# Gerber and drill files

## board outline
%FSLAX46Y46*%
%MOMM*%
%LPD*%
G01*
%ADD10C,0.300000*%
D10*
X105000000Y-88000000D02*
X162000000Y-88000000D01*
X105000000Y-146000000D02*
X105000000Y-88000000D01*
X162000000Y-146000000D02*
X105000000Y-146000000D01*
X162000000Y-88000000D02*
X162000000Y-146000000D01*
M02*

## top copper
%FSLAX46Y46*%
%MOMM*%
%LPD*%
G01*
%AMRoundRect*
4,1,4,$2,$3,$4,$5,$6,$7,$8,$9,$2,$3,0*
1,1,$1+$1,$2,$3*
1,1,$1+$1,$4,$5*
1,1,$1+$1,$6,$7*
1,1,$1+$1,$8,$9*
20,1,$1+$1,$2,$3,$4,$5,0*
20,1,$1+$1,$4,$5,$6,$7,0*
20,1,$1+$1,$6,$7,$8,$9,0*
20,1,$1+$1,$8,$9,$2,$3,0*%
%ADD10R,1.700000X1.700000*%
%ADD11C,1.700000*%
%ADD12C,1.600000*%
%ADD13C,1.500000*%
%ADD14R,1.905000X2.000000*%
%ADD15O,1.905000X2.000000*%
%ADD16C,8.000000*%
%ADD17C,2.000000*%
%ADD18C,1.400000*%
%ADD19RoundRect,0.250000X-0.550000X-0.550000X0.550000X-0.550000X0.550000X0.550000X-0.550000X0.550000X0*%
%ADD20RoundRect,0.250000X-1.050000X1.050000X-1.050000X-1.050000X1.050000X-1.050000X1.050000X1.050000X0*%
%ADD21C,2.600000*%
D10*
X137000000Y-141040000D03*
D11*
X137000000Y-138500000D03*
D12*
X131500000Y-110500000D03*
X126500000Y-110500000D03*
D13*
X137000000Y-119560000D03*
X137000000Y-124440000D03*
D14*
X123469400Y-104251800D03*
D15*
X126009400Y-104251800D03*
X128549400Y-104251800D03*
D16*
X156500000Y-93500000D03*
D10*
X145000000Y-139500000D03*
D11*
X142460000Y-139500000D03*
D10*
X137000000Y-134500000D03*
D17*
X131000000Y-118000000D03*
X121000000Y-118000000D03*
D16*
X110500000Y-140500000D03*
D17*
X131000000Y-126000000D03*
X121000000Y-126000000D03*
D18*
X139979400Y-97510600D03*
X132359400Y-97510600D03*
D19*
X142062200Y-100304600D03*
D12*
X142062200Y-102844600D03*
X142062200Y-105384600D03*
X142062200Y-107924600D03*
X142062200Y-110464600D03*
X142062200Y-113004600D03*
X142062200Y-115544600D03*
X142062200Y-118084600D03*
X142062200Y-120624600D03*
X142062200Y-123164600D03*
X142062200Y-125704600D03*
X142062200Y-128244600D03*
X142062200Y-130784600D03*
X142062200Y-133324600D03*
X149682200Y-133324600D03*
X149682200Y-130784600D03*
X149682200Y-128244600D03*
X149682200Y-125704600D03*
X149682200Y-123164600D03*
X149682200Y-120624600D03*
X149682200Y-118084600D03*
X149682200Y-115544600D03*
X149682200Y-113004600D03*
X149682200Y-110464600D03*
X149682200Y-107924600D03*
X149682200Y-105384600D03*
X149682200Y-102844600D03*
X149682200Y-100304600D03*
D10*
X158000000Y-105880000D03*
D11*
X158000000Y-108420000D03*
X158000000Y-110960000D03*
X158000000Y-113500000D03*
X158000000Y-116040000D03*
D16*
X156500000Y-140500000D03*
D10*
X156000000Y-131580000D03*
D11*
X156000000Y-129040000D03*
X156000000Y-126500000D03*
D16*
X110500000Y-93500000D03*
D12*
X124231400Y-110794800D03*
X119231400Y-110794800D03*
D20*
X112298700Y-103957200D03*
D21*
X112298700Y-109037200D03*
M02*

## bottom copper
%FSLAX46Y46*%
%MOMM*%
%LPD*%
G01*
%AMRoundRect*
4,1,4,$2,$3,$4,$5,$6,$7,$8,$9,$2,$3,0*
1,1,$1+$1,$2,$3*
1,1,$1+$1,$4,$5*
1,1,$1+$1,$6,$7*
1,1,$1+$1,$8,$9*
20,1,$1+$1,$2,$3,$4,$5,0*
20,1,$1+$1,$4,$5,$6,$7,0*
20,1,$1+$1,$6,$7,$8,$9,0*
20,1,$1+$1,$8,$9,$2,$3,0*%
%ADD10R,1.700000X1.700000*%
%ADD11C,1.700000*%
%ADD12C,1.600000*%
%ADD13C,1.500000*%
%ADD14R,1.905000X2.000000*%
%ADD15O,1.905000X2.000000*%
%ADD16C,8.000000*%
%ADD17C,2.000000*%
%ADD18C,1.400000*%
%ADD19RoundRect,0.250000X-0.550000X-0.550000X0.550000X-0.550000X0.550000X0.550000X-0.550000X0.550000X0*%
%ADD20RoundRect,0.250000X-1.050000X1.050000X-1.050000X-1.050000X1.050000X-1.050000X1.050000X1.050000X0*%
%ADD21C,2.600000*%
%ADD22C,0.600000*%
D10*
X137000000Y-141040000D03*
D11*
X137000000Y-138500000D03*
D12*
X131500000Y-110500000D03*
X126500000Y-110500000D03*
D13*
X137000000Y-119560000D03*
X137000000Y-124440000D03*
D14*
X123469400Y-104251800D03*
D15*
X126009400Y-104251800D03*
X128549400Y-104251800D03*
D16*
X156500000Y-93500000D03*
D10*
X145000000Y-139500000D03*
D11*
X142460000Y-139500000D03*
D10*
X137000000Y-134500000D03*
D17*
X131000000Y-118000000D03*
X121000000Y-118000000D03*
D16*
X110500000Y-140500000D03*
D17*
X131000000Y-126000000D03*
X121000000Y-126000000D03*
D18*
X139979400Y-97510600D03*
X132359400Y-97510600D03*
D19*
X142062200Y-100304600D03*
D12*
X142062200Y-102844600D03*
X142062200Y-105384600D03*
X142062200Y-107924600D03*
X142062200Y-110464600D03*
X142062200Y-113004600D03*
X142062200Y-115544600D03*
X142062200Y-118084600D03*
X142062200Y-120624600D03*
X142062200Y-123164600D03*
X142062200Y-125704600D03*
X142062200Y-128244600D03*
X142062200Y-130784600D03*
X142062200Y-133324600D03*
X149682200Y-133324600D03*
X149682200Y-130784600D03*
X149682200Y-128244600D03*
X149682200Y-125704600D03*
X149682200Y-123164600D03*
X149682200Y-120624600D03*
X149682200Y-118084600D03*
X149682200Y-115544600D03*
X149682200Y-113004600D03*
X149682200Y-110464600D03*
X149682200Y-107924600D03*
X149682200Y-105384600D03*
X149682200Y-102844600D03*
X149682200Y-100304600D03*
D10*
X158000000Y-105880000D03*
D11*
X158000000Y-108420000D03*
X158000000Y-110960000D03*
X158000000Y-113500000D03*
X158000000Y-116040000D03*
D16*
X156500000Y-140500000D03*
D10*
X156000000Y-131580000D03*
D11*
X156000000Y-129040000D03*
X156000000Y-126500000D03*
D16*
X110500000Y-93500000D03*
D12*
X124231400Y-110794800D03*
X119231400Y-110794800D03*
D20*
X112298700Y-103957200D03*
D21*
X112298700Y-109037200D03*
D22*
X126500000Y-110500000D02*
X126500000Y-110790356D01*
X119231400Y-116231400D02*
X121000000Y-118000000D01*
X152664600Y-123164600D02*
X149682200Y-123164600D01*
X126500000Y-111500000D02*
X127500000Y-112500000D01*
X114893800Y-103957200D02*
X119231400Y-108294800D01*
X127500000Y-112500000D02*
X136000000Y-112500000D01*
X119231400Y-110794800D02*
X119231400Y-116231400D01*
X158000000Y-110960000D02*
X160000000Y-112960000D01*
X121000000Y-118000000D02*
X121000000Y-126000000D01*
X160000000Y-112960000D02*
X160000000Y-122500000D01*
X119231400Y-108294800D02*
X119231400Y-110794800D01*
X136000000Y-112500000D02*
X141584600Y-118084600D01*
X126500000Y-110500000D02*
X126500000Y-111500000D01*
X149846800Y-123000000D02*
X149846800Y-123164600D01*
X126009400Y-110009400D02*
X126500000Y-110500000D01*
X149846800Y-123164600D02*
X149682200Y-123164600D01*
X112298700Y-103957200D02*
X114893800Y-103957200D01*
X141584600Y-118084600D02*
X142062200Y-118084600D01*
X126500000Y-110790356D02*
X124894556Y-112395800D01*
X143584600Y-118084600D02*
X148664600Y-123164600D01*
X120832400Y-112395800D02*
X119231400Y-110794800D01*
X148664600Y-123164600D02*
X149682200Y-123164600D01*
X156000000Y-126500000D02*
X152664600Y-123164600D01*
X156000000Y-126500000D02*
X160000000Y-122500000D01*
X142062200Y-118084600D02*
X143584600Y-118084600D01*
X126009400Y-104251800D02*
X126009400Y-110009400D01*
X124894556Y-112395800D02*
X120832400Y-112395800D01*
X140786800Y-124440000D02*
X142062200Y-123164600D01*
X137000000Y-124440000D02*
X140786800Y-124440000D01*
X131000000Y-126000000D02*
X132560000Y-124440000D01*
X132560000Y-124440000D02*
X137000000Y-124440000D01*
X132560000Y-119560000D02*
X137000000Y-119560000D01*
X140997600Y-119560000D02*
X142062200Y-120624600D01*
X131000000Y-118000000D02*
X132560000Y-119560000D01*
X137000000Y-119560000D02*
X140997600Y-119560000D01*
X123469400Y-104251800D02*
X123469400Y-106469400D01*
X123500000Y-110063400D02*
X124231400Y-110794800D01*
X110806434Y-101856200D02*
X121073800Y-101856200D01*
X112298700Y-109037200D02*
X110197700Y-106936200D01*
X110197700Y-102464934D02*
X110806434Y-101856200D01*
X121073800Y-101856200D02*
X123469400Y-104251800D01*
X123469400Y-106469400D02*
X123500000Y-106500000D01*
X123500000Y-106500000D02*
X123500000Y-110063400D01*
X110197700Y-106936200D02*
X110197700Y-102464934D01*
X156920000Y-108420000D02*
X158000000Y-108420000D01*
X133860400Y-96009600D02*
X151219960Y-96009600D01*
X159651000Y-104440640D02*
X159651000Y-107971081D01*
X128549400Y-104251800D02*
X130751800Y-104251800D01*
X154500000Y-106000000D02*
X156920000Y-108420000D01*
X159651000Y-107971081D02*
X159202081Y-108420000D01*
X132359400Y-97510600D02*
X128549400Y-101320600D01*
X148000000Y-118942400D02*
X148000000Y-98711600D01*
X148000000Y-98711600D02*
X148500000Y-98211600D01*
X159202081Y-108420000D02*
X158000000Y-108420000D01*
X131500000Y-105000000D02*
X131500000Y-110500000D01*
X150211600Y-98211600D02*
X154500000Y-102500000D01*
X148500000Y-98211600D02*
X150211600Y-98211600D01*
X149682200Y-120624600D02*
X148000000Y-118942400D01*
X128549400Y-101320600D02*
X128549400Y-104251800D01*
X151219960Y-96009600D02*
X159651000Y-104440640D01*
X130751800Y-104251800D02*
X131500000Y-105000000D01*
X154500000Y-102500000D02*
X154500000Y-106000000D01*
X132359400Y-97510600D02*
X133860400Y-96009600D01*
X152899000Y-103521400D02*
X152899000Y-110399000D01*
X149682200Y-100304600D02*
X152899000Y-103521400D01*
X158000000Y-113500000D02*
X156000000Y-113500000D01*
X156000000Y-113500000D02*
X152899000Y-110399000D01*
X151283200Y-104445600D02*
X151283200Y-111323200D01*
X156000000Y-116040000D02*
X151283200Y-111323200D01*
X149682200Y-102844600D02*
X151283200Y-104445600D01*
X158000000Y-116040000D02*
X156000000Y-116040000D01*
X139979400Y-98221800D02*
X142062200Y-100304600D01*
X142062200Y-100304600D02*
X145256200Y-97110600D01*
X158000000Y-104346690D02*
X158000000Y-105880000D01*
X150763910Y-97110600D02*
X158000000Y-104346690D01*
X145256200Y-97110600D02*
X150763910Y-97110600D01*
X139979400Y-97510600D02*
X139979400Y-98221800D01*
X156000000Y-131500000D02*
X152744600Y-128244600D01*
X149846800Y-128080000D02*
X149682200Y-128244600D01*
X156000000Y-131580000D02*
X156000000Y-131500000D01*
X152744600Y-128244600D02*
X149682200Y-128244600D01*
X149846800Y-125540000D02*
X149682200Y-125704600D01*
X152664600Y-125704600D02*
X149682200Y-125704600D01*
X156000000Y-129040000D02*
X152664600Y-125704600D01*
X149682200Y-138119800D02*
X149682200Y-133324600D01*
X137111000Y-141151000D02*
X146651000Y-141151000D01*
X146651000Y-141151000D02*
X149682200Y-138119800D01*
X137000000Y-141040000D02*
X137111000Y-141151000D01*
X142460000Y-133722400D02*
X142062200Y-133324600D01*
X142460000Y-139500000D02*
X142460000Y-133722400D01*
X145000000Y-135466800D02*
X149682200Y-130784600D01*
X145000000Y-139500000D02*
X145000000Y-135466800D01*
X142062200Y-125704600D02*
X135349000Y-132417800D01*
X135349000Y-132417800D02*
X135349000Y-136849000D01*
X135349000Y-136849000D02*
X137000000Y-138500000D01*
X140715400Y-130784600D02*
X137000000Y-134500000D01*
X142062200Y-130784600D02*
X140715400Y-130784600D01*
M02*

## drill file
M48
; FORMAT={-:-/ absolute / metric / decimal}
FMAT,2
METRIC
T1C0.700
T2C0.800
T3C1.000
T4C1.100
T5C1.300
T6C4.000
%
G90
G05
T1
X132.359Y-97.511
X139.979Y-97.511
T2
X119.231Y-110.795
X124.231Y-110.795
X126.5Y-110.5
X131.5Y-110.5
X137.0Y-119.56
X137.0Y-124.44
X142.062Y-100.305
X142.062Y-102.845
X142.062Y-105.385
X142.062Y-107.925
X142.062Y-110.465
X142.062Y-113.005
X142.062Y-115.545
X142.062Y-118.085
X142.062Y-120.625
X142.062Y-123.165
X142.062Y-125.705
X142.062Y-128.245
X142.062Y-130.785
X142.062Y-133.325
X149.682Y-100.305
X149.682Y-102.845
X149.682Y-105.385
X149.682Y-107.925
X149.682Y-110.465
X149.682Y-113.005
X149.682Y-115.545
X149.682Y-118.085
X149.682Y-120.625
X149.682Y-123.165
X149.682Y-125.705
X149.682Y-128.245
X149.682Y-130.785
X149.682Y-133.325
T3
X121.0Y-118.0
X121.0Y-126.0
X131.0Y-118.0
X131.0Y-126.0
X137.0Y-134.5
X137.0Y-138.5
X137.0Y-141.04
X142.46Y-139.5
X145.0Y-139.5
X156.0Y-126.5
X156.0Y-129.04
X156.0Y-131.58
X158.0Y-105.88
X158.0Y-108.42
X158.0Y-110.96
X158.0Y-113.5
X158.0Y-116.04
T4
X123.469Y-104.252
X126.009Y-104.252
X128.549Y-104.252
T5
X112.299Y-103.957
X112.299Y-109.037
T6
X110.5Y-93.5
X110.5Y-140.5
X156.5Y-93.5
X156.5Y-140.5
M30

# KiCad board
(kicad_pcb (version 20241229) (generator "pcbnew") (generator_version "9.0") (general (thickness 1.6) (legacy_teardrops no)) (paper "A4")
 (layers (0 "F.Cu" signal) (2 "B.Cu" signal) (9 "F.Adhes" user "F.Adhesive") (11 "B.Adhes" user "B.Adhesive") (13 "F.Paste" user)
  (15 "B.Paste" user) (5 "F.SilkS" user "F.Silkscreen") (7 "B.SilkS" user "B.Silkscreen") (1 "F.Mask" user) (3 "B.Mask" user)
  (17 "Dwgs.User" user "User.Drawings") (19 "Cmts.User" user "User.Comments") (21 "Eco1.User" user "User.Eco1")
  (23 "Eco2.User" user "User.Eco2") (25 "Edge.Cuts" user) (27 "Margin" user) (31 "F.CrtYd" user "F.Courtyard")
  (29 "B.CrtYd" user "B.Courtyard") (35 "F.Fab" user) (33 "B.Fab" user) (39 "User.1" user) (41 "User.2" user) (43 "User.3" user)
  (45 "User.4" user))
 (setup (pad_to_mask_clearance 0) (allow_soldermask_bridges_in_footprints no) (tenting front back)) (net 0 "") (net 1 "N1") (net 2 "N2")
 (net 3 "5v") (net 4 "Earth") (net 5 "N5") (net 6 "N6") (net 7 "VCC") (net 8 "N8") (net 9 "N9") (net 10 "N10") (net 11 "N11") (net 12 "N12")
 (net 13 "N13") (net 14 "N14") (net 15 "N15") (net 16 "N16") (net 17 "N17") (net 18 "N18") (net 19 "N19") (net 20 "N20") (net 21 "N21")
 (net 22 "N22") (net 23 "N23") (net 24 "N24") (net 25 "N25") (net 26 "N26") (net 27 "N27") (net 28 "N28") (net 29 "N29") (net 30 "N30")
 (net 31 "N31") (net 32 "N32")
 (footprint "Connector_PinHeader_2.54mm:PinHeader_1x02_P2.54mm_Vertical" (layer "F.Cu") (at 137 141.04 180)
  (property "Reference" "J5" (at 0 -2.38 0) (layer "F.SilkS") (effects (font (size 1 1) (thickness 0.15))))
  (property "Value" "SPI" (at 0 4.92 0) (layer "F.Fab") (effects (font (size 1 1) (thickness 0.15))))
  (pad "1" thru_hole rect (at 0 0 180) (size 1.7 1.7) (drill 1) (layers "*.Cu" "*.Mask") (remove_unused_layers no) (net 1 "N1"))
  (pad "2" thru_hole circle (at 0 2.54 180) (size 1.7 1.7) (drill 1) (layers "*.Cu" "*.Mask") (remove_unused_layers no) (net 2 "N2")))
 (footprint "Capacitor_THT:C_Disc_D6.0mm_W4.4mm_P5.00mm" (layer "F.Cu") (at 131.5 110.5 180)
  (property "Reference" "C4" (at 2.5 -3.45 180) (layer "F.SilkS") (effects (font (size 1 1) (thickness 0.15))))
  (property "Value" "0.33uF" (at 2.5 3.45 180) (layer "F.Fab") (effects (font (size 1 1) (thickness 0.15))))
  (pad "1" thru_hole circle (at 0 0 180) (size 1.6 1.6) (drill 0.8) (layers "*.Cu" "*.Mask") (remove_unused_layers no) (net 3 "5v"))
  (pad "2" thru_hole circle (at 5 0 180) (size 1.6 1.6) (drill 0.8) (layers "*.Cu" "*.Mask") (remove_unused_layers no) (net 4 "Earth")))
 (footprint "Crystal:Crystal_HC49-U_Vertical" (layer "F.Cu") (at 137 119.56 -90)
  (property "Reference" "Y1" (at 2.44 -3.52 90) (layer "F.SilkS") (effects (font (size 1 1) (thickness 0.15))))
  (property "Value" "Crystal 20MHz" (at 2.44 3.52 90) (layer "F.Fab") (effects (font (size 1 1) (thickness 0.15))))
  (pad "1" thru_hole circle (at 0 0 270) (size 1.5 1.5) (drill 0.8) (layers "*.Cu" "*.Mask") (remove_unused_layers no) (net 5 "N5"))
  (pad "2" thru_hole circle (at 4.88 0 270) (size 1.5 1.5) (drill 0.8) (layers "*.Cu" "*.Mask") (remove_unused_layers no) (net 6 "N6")))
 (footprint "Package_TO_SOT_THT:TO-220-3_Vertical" (layer "F.Cu") (at 123.4694 104.2518)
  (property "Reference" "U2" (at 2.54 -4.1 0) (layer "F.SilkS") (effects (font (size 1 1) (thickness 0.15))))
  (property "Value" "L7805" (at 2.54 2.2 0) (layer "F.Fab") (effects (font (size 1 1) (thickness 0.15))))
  (pad "1" thru_hole rect (at 0 0) (size 1.905 2) (drill 1.1) (layers "*.Cu" "*.Mask") (remove_unused_layers no) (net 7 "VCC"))
  (pad "2" thru_hole oval (at 2.54 0) (size 1.905 2) (drill 1.1) (layers "*.Cu" "*.Mask") (remove_unused_layers no) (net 4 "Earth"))
  (pad "3" thru_hole oval (at 5.08 0) (size 1.905 2) (drill 1.1) (layers "*.Cu" "*.Mask") (remove_unused_layers no) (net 3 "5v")))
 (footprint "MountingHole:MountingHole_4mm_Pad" (layer "F.Cu") (at 156.5 93.5)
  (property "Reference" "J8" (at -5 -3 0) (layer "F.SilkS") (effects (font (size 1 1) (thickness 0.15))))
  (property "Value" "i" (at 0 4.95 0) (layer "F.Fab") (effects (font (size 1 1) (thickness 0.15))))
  (pad "1" thru_hole circle (at 0 0) (size 8 8) (drill 4) (layers "*.Cu" "*.Mask") (remove_unused_layers no) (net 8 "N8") (zone_connect 2)))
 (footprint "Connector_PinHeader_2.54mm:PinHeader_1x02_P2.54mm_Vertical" (layer "F.Cu") (at 145 139.5 -90)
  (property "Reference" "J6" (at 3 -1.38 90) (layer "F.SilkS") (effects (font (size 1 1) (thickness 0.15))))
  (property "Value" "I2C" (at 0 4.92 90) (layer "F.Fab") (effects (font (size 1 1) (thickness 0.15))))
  (pad "1" thru_hole rect (at 0 0 270) (size 1.7 1.7) (drill 1) (layers "*.Cu" "*.Mask") (remove_unused_layers no) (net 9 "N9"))
  (pad "2" thru_hole circle (at 0 2.54 270) (size 1.7 1.7) (drill 1) (layers "*.Cu" "*.Mask") (remove_unused_layers no) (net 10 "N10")))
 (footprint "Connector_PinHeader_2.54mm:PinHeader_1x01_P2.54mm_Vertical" (layer "F.Cu") (at 137 134.5)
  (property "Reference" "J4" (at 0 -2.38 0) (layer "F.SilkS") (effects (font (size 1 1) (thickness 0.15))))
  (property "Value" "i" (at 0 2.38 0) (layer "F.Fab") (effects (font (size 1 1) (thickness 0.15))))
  (pad "1" thru_hole rect (at 0 0) (size 1.7 1.7) (drill 1) (layers "*.Cu" "*.Mask") (remove_unused_layers no) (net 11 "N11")))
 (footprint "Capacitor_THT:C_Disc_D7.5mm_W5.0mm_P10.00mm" (layer "F.Cu") (at 131 118 180)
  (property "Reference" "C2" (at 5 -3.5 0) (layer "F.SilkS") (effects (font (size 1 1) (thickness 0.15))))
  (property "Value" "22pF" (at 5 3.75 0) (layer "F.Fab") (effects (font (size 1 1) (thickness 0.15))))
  (pad "1" thru_hole circle (at 0 0 180) (size 2 2) (drill 1) (layers "*.Cu" "*.Mask") (remove_unused_layers no) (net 5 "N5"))
  (pad "2" thru_hole circle (at 10 0 180) (size 2 2) (drill 1) (layers "*.Cu" "*.Mask") (remove_unused_layers no) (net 4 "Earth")))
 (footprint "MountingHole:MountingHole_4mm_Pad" (layer "F.Cu") (at 110.5 140.5)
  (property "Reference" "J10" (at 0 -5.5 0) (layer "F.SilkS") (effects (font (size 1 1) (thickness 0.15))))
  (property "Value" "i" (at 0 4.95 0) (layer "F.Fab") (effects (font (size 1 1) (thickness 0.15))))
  (pad "1" thru_hole circle (at 0 0) (size 8 8) (drill 4) (layers "*.Cu" "*.Mask") (remove_unused_layers no) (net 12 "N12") (zone_connect 2)))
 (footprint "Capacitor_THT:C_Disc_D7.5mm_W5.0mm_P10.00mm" (layer "F.Cu") (at 131 126 180)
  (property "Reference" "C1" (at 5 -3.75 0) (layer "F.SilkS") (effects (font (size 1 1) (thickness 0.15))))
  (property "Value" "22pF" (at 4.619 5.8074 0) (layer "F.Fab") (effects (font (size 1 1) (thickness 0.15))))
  (pad "1" thru_hole circle (at 0 0 180) (size 2 2) (drill 1) (layers "*.Cu" "*.Mask") (remove_unused_layers no) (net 6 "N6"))
  (pad "2" thru_hole circle (at 10 0 180) (size 2 2) (drill 1) (layers "*.Cu" "*.Mask") (remove_unused_layers no) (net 4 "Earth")))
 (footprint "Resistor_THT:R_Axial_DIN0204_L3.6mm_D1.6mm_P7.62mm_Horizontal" (layer "F.Cu") (at 139.9794 97.5106 180)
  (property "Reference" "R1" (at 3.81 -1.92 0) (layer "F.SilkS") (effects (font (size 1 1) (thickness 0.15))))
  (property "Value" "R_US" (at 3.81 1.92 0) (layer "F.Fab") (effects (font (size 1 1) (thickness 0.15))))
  (pad "1" thru_hole circle (at 0 0 180) (size 1.4 1.4) (drill 0.7) (layers "*.Cu" "*.Mask") (remove_unused_layers no) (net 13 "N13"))
  (pad "2" thru_hole circle (at 7.62 0 180) (size 1.4 1.4) (drill 0.7) (layers "*.Cu" "*.Mask") (remove_unused_layers no) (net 3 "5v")))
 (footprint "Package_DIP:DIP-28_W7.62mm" (layer "F.Cu") (at 142.0622 100.3046)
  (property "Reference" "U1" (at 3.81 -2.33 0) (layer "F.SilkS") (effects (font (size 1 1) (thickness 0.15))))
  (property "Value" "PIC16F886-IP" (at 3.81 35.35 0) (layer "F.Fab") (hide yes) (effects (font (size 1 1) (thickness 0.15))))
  (pad "1" thru_hole roundrect (at 0 0) (size 1.6 1.6) (drill 0.8) (layers "*.Cu" "*.Mask") (remove_unused_layers no)
   (roundrect_rratio 0.15625) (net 13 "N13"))
  (pad "2" thru_hole circle (at 0 2.54) (size 1.6 1.6) (drill 0.8) (layers "*.Cu" "*.Mask") (remove_unused_layers no) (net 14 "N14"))
  (pad "3" thru_hole circle (at 0 5.08) (size 1.6 1.6) (drill 0.8) (layers "*.Cu" "*.Mask") (remove_unused_layers no) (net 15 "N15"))
  (pad "4" thru_hole circle (at 0 7.62) (size 1.6 1.6) (drill 0.8) (layers "*.Cu" "*.Mask") (remove_unused_layers no) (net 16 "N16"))
  (pad "5" thru_hole circle (at 0 10.16) (size 1.6 1.6) (drill 0.8) (layers "*.Cu" "*.Mask") (remove_unused_layers no) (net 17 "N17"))
  (pad "6" thru_hole circle (at 0 12.7) (size 1.6 1.6) (drill 0.8) (layers "*.Cu" "*.Mask") (remove_unused_layers no) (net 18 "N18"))
  (pad "7" thru_hole circle (at 0 15.24) (size 1.6 1.6) (drill 0.8) (layers "*.Cu" "*.Mask") (remove_unused_layers no) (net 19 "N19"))
  (pad "8" thru_hole circle (at 0 17.78) (size 1.6 1.6) (drill 0.8) (layers "*.Cu" "*.Mask") (remove_unused_layers no) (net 4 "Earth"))
  (pad "9" thru_hole circle (at 0 20.32) (size 1.6 1.6) (drill 0.8) (layers "*.Cu" "*.Mask") (remove_unused_layers no) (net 5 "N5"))
  (pad "10" thru_hole circle (at 0 22.86) (size 1.6 1.6) (drill 0.8) (layers "*.Cu" "*.Mask") (remove_unused_layers no) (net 6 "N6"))
  (pad "11" thru_hole circle (at 0 25.4) (size 1.6 1.6) (drill 0.8) (layers "*.Cu" "*.Mask") (remove_unused_layers no) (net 2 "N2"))
  (pad "12" thru_hole circle (at 0 27.94) (size 1.6 1.6) (drill 0.8) (layers "*.Cu" "*.Mask") (remove_unused_layers no) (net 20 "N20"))
  (pad "13" thru_hole circle (at 0 30.48) (size 1.6 1.6) (drill 0.8) (layers "*.Cu" "*.Mask") (remove_unused_layers no) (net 11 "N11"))
  (pad "14" thru_hole circle (at 0 33.02) (size 1.6 1.6) (drill 0.8) (layers "*.Cu" "*.Mask") (remove_unused_layers no) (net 10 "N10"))
  (pad "15" thru_hole circle (at 7.62 33.02) (size 1.6 1.6) (drill 0.8) (layers "*.Cu" "*.Mask") (remove_unused_layers no) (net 1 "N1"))
  (pad "16" thru_hole circle (at 7.62 30.48) (size 1.6 1.6) (drill 0.8) (layers "*.Cu" "*.Mask") (remove_unused_layers no) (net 9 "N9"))
  (pad "17" thru_hole circle (at 7.62 27.94) (size 1.6 1.6) (drill 0.8) (layers "*.Cu" "*.Mask") (remove_unused_layers no) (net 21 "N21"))
  (pad "18" thru_hole circle (at 7.62 25.4) (size 1.6 1.6) (drill 0.8) (layers "*.Cu" "*.Mask") (remove_unused_layers no) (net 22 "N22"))
  (pad "19" thru_hole circle (at 7.62 22.86) (size 1.6 1.6) (drill 0.8) (layers "*.Cu" "*.Mask") (remove_unused_layers no) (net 4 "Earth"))
  (pad "20" thru_hole circle (at 7.62 20.32) (size 1.6 1.6) (drill 0.8) (layers "*.Cu" "*.Mask") (remove_unused_layers no) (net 3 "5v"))
  (pad "21" thru_hole circle (at 7.62 17.78) (size 1.6 1.6) (drill 0.8) (layers "*.Cu" "*.Mask") (remove_unused_layers no) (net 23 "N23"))
  (pad "22" thru_hole circle (at 7.62 15.24) (size 1.6 1.6) (drill 0.8) (layers "*.Cu" "*.Mask") (remove_unused_layers no) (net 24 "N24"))
  (pad "23" thru_hole circle (at 7.62 12.7) (size 1.6 1.6) (drill 0.8) (layers "*.Cu" "*.Mask") (remove_unused_layers no) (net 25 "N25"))
  (pad "24" thru_hole circle (at 7.62 10.16) (size 1.6 1.6) (drill 0.8) (layers "*.Cu" "*.Mask") (remove_unused_layers no) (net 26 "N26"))
  (pad "25" thru_hole circle (at 7.62 7.62) (size 1.6 1.6) (drill 0.8) (layers "*.Cu" "*.Mask") (remove_unused_layers no) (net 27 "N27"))
  (pad "26" thru_hole circle (at 7.62 5.08) (size 1.6 1.6) (drill 0.8) (layers "*.Cu" "*.Mask") (remove_unused_layers no) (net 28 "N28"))
  (pad "27" thru_hole circle (at 7.62 2.54) (size 1.6 1.6) (drill 0.8) (layers "*.Cu" "*.Mask") (remove_unused_layers no) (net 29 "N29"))
  (pad "28" thru_hole circle (at 7.62 0) (size 1.6 1.6) (drill 0.8) (layers "*.Cu" "*.Mask") (remove_unused_layers no) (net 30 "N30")))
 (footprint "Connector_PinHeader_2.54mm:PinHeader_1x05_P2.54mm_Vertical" (layer "F.Cu") (at 158 105.88)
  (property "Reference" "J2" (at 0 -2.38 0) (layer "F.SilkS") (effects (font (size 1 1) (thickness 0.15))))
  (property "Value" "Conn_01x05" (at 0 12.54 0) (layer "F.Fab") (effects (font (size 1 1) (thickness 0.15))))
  (pad "1" thru_hole rect (at 0 0) (size 1.7 1.7) (drill 1) (layers "*.Cu" "*.Mask") (remove_unused_layers no) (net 13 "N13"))
  (pad "2" thru_hole circle (at 0 2.54) (size 1.7 1.7) (drill 1) (layers "*.Cu" "*.Mask") (remove_unused_layers no) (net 3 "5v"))
  (pad "3" thru_hole circle (at 0 5.08) (size 1.7 1.7) (drill 1) (layers "*.Cu" "*.Mask") (remove_unused_layers no) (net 4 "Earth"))
  (pad "4" thru_hole circle (at 0 7.62) (size 1.7 1.7) (drill 1) (layers "*.Cu" "*.Mask") (remove_unused_layers no) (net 30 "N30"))
  (pad "5" thru_hole circle (at 0 10.16) (size 1.7 1.7) (drill 1) (layers "*.Cu" "*.Mask") (remove_unused_layers no) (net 29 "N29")))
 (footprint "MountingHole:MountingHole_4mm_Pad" (layer "F.Cu") (at 156.5 140.5)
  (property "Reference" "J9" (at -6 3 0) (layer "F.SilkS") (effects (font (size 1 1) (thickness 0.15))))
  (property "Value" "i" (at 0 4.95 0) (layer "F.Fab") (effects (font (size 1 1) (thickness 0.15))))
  (pad "1" thru_hole circle (at 0 0) (size 8 8) (drill 4) (layers "*.Cu" "*.Mask") (remove_unused_layers no) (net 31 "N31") (zone_connect 2)))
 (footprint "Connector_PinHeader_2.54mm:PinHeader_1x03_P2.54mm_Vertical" (layer "F.Cu") (at 156 131.58 180)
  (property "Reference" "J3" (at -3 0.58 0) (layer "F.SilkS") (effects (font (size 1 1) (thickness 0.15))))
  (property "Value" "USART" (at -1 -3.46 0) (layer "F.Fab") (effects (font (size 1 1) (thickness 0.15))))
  (pad "1" thru_hole rect (at 0 0 180) (size 1.7 1.7) (drill 1) (layers "*.Cu" "*.Mask") (remove_unused_layers no) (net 21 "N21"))
  (pad "2" thru_hole circle (at 0 2.54 180) (size 1.7 1.7) (drill 1) (layers "*.Cu" "*.Mask") (remove_unused_layers no) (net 22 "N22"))
  (pad "3" thru_hole circle (at 0 5.08 180) (size 1.7 1.7) (drill 1) (layers "*.Cu" "*.Mask") (remove_unused_layers no) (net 4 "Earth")))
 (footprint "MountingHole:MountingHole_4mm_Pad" (layer "F.Cu") (at 110.5 93.5)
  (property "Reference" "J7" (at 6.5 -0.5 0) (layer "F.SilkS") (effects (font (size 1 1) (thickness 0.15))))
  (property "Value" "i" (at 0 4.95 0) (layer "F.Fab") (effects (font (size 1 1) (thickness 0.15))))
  (pad "1" thru_hole circle (at 0 0) (size 8 8) (drill 4) (layers "*.Cu" "*.Mask") (remove_unused_layers no) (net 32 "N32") (zone_connect 2)))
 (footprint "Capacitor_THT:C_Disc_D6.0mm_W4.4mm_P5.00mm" (layer "F.Cu") (at 124.2314 110.7948 180)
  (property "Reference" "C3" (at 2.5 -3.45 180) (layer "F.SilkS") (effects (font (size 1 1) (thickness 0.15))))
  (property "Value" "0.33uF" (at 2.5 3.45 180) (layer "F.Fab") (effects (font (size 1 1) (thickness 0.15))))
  (pad "1" thru_hole circle (at 0 0 180) (size 1.6 1.6) (drill 0.8) (layers "*.Cu" "*.Mask") (remove_unused_layers no) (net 7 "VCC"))
  (pad "2" thru_hole circle (at 5 0 180) (size 1.6 1.6) (drill 0.8) (layers "*.Cu" "*.Mask") (remove_unused_layers no) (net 4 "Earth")))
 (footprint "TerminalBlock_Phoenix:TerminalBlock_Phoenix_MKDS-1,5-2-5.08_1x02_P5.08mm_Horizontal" (layer "F.Cu") (at 112.2987 103.9572 -90)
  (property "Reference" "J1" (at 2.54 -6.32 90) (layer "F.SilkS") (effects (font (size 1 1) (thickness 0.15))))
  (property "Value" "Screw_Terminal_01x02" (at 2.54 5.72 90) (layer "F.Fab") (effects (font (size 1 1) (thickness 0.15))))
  (pad "1" thru_hole roundrect (at 0 0 270) (size 2.6 2.6) (drill 1.3) (layers "*.Cu" "*.Mask") (remove_unused_layers no)
   (roundrect_rratio 0.096154) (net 4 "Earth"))
  (pad "2" thru_hole circle (at 5.08 0 270) (size 2.6 2.6) (drill 1.3) (layers "*.Cu" "*.Mask") (remove_unused_layers no) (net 7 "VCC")))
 (gr_line (start 105 88) (end 162 88) (stroke (width 0.3) (type default)) (layer "Edge.Cuts"))
 (gr_line (start 105 146) (end 105 88) (stroke (width 0.3) (type default)) (layer "Edge.Cuts"))
 (gr_line (start 162 146) (end 105 146) (stroke (width 0.3) (type default)) (layer "Edge.Cuts"))
 (gr_line (start 162 88) (end 162 146) (stroke (width 0.3) (type default)) (layer "Edge.Cuts"))
 (segment (start 126.5 110.5) (end 126.5 110.790356) (width 0.6) (layer "B.Cu") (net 4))
 (segment (start 119.2314 116.2314) (end 121 118) (width 0.6) (layer "B.Cu") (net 4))
 (segment (start 152.6646 123.1646) (end 149.6822 123.1646) (width 0.6) (layer "B.Cu") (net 4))
 (segment (start 126.5 111.5) (end 127.5 112.5) (width 0.6) (layer "B.Cu") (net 4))
 (segment (start 114.8938 103.9572) (end 119.2314 108.2948) (width 0.6) (layer "B.Cu") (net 4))
 (segment (start 127.5 112.5) (end 136 112.5) (width 0.6) (layer "B.Cu") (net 4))
 (segment (start 119.2314 110.7948) (end 119.2314 116.2314) (width 0.6) (layer "B.Cu") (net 4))
 (segment (start 158 110.96) (end 160 112.96) (width 0.6) (layer "B.Cu") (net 4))
 (segment (start 121 118) (end 121 126) (width 0.6) (layer "B.Cu") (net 4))
 (segment (start 160 112.96) (end 160 122.5) (width 0.6) (layer "B.Cu") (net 4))
 (segment (start 119.2314 108.2948) (end 119.2314 110.7948) (width 0.6) (layer "B.Cu") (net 4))
 (segment (start 136 112.5) (end 141.5846 118.0846) (width 0.6) (layer "B.Cu") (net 4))
 (segment (start 126.5 110.5) (end 126.5 111.5) (width 0.6) (layer "B.Cu") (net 4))
 (segment (start 149.8468 123) (end 149.8468 123.1646) (width 0.6) (layer "B.Cu") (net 4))
 (segment (start 126.0094 110.0094) (end 126.5 110.5) (width 0.6) (layer "B.Cu") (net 4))
 (segment (start 149.8468 123.1646) (end 149.6822 123.1646) (width 0.6) (layer "B.Cu") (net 4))
 (segment (start 112.2987 103.9572) (end 114.8938 103.9572) (width 0.6) (layer "B.Cu") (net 4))
 (segment (start 141.5846 118.0846) (end 142.0622 118.0846) (width 0.6) (layer "B.Cu") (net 4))
 (segment (start 126.5 110.790356) (end 124.894556 112.3958) (width 0.6) (layer "B.Cu") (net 4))
 (segment (start 143.5846 118.0846) (end 148.6646 123.1646) (width 0.6) (layer "B.Cu") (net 4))
 (segment (start 120.8324 112.3958) (end 119.2314 110.7948) (width 0.6) (layer "B.Cu") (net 4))
 (segment (start 148.6646 123.1646) (end 149.6822 123.1646) (width 0.6) (layer "B.Cu") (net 4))
 (segment (start 156 126.5) (end 152.6646 123.1646) (width 0.6) (layer "B.Cu") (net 4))
 (segment (start 156 126.5) (end 160 122.5) (width 0.6) (layer "B.Cu") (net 4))
 (segment (start 142.0622 118.0846) (end 143.5846 118.0846) (width 0.6) (layer "B.Cu") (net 4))
 (segment (start 126.0094 104.2518) (end 126.0094 110.0094) (width 0.6) (layer "B.Cu") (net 4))
 (segment (start 124.894556 112.3958) (end 120.8324 112.3958) (width 0.6) (layer "B.Cu") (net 4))
 (segment (start 140.7868 124.44) (end 142.0622 123.1646) (width 0.6) (layer "B.Cu") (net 6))
 (segment (start 137 124.44) (end 140.7868 124.44) (width 0.6) (layer "B.Cu") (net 6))
 (segment (start 131 126) (end 132.56 124.44) (width 0.6) (layer "B.Cu") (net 6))
 (segment (start 132.56 124.44) (end 137 124.44) (width 0.6) (layer "B.Cu") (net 6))
 (segment (start 132.56 119.56) (end 137 119.56) (width 0.6) (layer "B.Cu") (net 5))
 (segment (start 140.9976 119.56) (end 142.0622 120.6246) (width 0.6) (layer "B.Cu") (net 5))
 (segment (start 131 118) (end 132.56 119.56) (width 0.6) (layer "B.Cu") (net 5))
 (segment (start 137 119.56) (end 140.9976 119.56) (width 0.6) (layer "B.Cu") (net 5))
 (segment (start 123.4694 104.2518) (end 123.4694 106.4694) (width 0.6) (layer "B.Cu") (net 7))
 (segment (start 123.5 110.0634) (end 124.2314 110.7948) (width 0.6) (layer "B.Cu") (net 7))
 (segment (start 110.806434 101.8562) (end 121.0738 101.8562) (width 0.6) (layer "B.Cu") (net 7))
 (segment (start 112.2987 109.0372) (end 110.1977 106.9362) (width 0.6) (layer "B.Cu") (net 7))
 (segment (start 110.1977 102.464934) (end 110.806434 101.8562) (width 0.6) (layer "B.Cu") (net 7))
 (segment (start 121.0738 101.8562) (end 123.4694 104.2518) (width 0.6) (layer "B.Cu") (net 7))
 (segment (start 123.4694 106.4694) (end 123.5 106.5) (width 0.6) (layer "B.Cu") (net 7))
 (segment (start 123.5 106.5) (end 123.5 110.0634) (width 0.6) (layer "B.Cu") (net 7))
 (segment (start 110.1977 106.9362) (end 110.1977 102.464934) (width 0.6) (layer "B.Cu") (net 7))
 (segment (start 156.92 108.42) (end 158 108.42) (width 0.6) (layer "B.Cu") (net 3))
 (segment (start 133.8604 96.0096) (end 151.21996 96.0096) (width 0.6) (layer "B.Cu") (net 3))
 (segment (start 159.651 104.44064) (end 159.651 107.971081) (width 0.6) (layer "B.Cu") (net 3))
 (segment (start 128.5494 104.2518) (end 130.7518 104.2518) (width 0.6) (layer "B.Cu") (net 3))
 (segment (start 154.5 106) (end 156.92 108.42) (width 0.6) (layer "B.Cu") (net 3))
 (segment (start 159.651 107.971081) (end 159.202081 108.42) (width 0.6) (layer "B.Cu") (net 3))
 (segment (start 132.3594 97.5106) (end 128.5494 101.3206) (width 0.6) (layer "B.Cu") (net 3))
 (segment (start 148 118.9424) (end 148 98.7116) (width 0.6) (layer "B.Cu") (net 3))
 (segment (start 148 98.7116) (end 148.5 98.2116) (width 0.6) (layer "B.Cu") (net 3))
 (segment (start 159.202081 108.42) (end 158 108.42) (width 0.6) (layer "B.Cu") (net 3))
 (segment (start 131.5 105) (end 131.5 110.5) (width 0.6) (layer "B.Cu") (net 3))
 (segment (start 150.2116 98.2116) (end 154.5 102.5) (width 0.6) (layer "B.Cu") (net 3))
 (segment (start 148.5 98.2116) (end 150.2116 98.2116) (width 0.6) (layer "B.Cu") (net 3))
 (segment (start 149.6822 120.6246) (end 148 118.9424) (width 0.6) (layer "B.Cu") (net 3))
 (segment (start 128.5494 101.3206) (end 128.5494 104.2518) (width 0.6) (layer "B.Cu") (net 3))
 (segment (start 151.21996 96.0096) (end 159.651 104.44064) (width 0.6) (layer "B.Cu") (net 3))
 (segment (start 130.7518 104.2518) (end 131.5 105) (width 0.6) (layer "B.Cu") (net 3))
 (segment (start 154.5 102.5) (end 154.5 106) (width 0.6) (layer "B.Cu") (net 3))
 (segment (start 132.3594 97.5106) (end 133.8604 96.0096) (width 0.6) (layer "B.Cu") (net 3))
 (segment (start 152.899 103.5214) (end 152.899 110.399) (width 0.6) (layer "B.Cu") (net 30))
 (segment (start 149.6822 100.3046) (end 152.899 103.5214) (width 0.6) (layer "B.Cu") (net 30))
 (segment (start 158 113.5) (end 156 113.5) (width 0.6) (layer "B.Cu") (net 30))
 (segment (start 156 113.5) (end 152.899 110.399) (width 0.6) (layer "B.Cu") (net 30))
 (segment (start 151.2832 104.4456) (end 151.2832 111.3232) (width 0.6) (layer "B.Cu") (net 29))
 (segment (start 156 116.04) (end 151.2832 111.3232) (width 0.6) (layer "B.Cu") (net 29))
 (segment (start 149.6822 102.8446) (end 151.2832 104.4456) (width 0.6) (layer "B.Cu") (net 29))
 (segment (start 158 116.04) (end 156 116.04) (width 0.6) (layer "B.Cu") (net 29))
 (segment (start 139.9794 98.2218) (end 142.0622 100.3046) (width 0.6) (layer "B.Cu") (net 13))
 (segment (start 142.0622 100.3046) (end 145.2562 97.1106) (width 0.6) (layer "B.Cu") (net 13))
 (segment (start 158 104.34669) (end 158 105.88) (width 0.6) (layer "B.Cu") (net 13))
 (segment (start 150.76391 97.1106) (end 158 104.34669) (width 0.6) (layer "B.Cu") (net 13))
 (segment (start 145.2562 97.1106) (end 150.76391 97.1106) (width 0.6) (layer "B.Cu") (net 13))
 (segment (start 139.9794 97.5106) (end 139.9794 98.2218) (width 0.6) (layer "B.Cu") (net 13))
 (segment (start 156 131.5) (end 152.7446 128.2446) (width 0.6) (layer "B.Cu") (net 21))
 (segment (start 149.8468 128.08) (end 149.6822 128.2446) (width 0.6) (layer "B.Cu") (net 21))
 (segment (start 156 131.58) (end 156 131.5) (width 0.6) (layer "B.Cu") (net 21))
 (segment (start 152.7446 128.2446) (end 149.6822 128.2446) (width 0.6) (layer "B.Cu") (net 21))
 (segment (start 149.8468 125.54) (end 149.6822 125.7046) (width 0.6) (layer "B.Cu") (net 22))
 (segment (start 152.6646 125.7046) (end 149.6822 125.7046) (width 0.6) (layer "B.Cu") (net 22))
 (segment (start 156 129.04) (end 152.6646 125.7046) (width 0.6) (layer "B.Cu") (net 22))
 (segment (start 149.6822 138.1198) (end 149.6822 133.3246) (width 0.6) (layer "B.Cu") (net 1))
 (segment (start 137.111 141.151) (end 146.651 141.151) (width 0.6) (layer "B.Cu") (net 1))
 (segment (start 146.651 141.151) (end 149.6822 138.1198) (width 0.6) (layer "B.Cu") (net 1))
 (segment (start 137 141.04) (end 137.111 141.151) (width 0.6) (layer "B.Cu") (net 1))
 (segment (start 142.46 133.7224) (end 142.0622 133.3246) (width 0.6) (layer "B.Cu") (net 10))
 (segment (start 142.46 139.5) (end 142.46 133.7224) (width 0.6) (layer "B.Cu") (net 10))
 (segment (start 145 135.4668) (end 149.6822 130.7846) (width 0.6) (layer "B.Cu") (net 9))
 (segment (start 145 139.5) (end 145 135.4668) (width 0.6) (layer "B.Cu") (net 9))
 (segment (start 142.0622 125.7046) (end 135.349 132.4178) (width 0.6) (layer "B.Cu") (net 2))
 (segment (start 135.349 132.4178) (end 135.349 136.849) (width 0.6) (layer "B.Cu") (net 2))
 (segment (start 135.349 136.849) (end 137 138.5) (width 0.6) (layer "B.Cu") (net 2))
 (segment (start 140.7154 130.7846) (end 137 134.5) (width 0.6) (layer "B.Cu") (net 11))
 (segment (start 142.0622 130.7846) (end 140.7154 130.7846) (width 0.6) (layer "B.Cu") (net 11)))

